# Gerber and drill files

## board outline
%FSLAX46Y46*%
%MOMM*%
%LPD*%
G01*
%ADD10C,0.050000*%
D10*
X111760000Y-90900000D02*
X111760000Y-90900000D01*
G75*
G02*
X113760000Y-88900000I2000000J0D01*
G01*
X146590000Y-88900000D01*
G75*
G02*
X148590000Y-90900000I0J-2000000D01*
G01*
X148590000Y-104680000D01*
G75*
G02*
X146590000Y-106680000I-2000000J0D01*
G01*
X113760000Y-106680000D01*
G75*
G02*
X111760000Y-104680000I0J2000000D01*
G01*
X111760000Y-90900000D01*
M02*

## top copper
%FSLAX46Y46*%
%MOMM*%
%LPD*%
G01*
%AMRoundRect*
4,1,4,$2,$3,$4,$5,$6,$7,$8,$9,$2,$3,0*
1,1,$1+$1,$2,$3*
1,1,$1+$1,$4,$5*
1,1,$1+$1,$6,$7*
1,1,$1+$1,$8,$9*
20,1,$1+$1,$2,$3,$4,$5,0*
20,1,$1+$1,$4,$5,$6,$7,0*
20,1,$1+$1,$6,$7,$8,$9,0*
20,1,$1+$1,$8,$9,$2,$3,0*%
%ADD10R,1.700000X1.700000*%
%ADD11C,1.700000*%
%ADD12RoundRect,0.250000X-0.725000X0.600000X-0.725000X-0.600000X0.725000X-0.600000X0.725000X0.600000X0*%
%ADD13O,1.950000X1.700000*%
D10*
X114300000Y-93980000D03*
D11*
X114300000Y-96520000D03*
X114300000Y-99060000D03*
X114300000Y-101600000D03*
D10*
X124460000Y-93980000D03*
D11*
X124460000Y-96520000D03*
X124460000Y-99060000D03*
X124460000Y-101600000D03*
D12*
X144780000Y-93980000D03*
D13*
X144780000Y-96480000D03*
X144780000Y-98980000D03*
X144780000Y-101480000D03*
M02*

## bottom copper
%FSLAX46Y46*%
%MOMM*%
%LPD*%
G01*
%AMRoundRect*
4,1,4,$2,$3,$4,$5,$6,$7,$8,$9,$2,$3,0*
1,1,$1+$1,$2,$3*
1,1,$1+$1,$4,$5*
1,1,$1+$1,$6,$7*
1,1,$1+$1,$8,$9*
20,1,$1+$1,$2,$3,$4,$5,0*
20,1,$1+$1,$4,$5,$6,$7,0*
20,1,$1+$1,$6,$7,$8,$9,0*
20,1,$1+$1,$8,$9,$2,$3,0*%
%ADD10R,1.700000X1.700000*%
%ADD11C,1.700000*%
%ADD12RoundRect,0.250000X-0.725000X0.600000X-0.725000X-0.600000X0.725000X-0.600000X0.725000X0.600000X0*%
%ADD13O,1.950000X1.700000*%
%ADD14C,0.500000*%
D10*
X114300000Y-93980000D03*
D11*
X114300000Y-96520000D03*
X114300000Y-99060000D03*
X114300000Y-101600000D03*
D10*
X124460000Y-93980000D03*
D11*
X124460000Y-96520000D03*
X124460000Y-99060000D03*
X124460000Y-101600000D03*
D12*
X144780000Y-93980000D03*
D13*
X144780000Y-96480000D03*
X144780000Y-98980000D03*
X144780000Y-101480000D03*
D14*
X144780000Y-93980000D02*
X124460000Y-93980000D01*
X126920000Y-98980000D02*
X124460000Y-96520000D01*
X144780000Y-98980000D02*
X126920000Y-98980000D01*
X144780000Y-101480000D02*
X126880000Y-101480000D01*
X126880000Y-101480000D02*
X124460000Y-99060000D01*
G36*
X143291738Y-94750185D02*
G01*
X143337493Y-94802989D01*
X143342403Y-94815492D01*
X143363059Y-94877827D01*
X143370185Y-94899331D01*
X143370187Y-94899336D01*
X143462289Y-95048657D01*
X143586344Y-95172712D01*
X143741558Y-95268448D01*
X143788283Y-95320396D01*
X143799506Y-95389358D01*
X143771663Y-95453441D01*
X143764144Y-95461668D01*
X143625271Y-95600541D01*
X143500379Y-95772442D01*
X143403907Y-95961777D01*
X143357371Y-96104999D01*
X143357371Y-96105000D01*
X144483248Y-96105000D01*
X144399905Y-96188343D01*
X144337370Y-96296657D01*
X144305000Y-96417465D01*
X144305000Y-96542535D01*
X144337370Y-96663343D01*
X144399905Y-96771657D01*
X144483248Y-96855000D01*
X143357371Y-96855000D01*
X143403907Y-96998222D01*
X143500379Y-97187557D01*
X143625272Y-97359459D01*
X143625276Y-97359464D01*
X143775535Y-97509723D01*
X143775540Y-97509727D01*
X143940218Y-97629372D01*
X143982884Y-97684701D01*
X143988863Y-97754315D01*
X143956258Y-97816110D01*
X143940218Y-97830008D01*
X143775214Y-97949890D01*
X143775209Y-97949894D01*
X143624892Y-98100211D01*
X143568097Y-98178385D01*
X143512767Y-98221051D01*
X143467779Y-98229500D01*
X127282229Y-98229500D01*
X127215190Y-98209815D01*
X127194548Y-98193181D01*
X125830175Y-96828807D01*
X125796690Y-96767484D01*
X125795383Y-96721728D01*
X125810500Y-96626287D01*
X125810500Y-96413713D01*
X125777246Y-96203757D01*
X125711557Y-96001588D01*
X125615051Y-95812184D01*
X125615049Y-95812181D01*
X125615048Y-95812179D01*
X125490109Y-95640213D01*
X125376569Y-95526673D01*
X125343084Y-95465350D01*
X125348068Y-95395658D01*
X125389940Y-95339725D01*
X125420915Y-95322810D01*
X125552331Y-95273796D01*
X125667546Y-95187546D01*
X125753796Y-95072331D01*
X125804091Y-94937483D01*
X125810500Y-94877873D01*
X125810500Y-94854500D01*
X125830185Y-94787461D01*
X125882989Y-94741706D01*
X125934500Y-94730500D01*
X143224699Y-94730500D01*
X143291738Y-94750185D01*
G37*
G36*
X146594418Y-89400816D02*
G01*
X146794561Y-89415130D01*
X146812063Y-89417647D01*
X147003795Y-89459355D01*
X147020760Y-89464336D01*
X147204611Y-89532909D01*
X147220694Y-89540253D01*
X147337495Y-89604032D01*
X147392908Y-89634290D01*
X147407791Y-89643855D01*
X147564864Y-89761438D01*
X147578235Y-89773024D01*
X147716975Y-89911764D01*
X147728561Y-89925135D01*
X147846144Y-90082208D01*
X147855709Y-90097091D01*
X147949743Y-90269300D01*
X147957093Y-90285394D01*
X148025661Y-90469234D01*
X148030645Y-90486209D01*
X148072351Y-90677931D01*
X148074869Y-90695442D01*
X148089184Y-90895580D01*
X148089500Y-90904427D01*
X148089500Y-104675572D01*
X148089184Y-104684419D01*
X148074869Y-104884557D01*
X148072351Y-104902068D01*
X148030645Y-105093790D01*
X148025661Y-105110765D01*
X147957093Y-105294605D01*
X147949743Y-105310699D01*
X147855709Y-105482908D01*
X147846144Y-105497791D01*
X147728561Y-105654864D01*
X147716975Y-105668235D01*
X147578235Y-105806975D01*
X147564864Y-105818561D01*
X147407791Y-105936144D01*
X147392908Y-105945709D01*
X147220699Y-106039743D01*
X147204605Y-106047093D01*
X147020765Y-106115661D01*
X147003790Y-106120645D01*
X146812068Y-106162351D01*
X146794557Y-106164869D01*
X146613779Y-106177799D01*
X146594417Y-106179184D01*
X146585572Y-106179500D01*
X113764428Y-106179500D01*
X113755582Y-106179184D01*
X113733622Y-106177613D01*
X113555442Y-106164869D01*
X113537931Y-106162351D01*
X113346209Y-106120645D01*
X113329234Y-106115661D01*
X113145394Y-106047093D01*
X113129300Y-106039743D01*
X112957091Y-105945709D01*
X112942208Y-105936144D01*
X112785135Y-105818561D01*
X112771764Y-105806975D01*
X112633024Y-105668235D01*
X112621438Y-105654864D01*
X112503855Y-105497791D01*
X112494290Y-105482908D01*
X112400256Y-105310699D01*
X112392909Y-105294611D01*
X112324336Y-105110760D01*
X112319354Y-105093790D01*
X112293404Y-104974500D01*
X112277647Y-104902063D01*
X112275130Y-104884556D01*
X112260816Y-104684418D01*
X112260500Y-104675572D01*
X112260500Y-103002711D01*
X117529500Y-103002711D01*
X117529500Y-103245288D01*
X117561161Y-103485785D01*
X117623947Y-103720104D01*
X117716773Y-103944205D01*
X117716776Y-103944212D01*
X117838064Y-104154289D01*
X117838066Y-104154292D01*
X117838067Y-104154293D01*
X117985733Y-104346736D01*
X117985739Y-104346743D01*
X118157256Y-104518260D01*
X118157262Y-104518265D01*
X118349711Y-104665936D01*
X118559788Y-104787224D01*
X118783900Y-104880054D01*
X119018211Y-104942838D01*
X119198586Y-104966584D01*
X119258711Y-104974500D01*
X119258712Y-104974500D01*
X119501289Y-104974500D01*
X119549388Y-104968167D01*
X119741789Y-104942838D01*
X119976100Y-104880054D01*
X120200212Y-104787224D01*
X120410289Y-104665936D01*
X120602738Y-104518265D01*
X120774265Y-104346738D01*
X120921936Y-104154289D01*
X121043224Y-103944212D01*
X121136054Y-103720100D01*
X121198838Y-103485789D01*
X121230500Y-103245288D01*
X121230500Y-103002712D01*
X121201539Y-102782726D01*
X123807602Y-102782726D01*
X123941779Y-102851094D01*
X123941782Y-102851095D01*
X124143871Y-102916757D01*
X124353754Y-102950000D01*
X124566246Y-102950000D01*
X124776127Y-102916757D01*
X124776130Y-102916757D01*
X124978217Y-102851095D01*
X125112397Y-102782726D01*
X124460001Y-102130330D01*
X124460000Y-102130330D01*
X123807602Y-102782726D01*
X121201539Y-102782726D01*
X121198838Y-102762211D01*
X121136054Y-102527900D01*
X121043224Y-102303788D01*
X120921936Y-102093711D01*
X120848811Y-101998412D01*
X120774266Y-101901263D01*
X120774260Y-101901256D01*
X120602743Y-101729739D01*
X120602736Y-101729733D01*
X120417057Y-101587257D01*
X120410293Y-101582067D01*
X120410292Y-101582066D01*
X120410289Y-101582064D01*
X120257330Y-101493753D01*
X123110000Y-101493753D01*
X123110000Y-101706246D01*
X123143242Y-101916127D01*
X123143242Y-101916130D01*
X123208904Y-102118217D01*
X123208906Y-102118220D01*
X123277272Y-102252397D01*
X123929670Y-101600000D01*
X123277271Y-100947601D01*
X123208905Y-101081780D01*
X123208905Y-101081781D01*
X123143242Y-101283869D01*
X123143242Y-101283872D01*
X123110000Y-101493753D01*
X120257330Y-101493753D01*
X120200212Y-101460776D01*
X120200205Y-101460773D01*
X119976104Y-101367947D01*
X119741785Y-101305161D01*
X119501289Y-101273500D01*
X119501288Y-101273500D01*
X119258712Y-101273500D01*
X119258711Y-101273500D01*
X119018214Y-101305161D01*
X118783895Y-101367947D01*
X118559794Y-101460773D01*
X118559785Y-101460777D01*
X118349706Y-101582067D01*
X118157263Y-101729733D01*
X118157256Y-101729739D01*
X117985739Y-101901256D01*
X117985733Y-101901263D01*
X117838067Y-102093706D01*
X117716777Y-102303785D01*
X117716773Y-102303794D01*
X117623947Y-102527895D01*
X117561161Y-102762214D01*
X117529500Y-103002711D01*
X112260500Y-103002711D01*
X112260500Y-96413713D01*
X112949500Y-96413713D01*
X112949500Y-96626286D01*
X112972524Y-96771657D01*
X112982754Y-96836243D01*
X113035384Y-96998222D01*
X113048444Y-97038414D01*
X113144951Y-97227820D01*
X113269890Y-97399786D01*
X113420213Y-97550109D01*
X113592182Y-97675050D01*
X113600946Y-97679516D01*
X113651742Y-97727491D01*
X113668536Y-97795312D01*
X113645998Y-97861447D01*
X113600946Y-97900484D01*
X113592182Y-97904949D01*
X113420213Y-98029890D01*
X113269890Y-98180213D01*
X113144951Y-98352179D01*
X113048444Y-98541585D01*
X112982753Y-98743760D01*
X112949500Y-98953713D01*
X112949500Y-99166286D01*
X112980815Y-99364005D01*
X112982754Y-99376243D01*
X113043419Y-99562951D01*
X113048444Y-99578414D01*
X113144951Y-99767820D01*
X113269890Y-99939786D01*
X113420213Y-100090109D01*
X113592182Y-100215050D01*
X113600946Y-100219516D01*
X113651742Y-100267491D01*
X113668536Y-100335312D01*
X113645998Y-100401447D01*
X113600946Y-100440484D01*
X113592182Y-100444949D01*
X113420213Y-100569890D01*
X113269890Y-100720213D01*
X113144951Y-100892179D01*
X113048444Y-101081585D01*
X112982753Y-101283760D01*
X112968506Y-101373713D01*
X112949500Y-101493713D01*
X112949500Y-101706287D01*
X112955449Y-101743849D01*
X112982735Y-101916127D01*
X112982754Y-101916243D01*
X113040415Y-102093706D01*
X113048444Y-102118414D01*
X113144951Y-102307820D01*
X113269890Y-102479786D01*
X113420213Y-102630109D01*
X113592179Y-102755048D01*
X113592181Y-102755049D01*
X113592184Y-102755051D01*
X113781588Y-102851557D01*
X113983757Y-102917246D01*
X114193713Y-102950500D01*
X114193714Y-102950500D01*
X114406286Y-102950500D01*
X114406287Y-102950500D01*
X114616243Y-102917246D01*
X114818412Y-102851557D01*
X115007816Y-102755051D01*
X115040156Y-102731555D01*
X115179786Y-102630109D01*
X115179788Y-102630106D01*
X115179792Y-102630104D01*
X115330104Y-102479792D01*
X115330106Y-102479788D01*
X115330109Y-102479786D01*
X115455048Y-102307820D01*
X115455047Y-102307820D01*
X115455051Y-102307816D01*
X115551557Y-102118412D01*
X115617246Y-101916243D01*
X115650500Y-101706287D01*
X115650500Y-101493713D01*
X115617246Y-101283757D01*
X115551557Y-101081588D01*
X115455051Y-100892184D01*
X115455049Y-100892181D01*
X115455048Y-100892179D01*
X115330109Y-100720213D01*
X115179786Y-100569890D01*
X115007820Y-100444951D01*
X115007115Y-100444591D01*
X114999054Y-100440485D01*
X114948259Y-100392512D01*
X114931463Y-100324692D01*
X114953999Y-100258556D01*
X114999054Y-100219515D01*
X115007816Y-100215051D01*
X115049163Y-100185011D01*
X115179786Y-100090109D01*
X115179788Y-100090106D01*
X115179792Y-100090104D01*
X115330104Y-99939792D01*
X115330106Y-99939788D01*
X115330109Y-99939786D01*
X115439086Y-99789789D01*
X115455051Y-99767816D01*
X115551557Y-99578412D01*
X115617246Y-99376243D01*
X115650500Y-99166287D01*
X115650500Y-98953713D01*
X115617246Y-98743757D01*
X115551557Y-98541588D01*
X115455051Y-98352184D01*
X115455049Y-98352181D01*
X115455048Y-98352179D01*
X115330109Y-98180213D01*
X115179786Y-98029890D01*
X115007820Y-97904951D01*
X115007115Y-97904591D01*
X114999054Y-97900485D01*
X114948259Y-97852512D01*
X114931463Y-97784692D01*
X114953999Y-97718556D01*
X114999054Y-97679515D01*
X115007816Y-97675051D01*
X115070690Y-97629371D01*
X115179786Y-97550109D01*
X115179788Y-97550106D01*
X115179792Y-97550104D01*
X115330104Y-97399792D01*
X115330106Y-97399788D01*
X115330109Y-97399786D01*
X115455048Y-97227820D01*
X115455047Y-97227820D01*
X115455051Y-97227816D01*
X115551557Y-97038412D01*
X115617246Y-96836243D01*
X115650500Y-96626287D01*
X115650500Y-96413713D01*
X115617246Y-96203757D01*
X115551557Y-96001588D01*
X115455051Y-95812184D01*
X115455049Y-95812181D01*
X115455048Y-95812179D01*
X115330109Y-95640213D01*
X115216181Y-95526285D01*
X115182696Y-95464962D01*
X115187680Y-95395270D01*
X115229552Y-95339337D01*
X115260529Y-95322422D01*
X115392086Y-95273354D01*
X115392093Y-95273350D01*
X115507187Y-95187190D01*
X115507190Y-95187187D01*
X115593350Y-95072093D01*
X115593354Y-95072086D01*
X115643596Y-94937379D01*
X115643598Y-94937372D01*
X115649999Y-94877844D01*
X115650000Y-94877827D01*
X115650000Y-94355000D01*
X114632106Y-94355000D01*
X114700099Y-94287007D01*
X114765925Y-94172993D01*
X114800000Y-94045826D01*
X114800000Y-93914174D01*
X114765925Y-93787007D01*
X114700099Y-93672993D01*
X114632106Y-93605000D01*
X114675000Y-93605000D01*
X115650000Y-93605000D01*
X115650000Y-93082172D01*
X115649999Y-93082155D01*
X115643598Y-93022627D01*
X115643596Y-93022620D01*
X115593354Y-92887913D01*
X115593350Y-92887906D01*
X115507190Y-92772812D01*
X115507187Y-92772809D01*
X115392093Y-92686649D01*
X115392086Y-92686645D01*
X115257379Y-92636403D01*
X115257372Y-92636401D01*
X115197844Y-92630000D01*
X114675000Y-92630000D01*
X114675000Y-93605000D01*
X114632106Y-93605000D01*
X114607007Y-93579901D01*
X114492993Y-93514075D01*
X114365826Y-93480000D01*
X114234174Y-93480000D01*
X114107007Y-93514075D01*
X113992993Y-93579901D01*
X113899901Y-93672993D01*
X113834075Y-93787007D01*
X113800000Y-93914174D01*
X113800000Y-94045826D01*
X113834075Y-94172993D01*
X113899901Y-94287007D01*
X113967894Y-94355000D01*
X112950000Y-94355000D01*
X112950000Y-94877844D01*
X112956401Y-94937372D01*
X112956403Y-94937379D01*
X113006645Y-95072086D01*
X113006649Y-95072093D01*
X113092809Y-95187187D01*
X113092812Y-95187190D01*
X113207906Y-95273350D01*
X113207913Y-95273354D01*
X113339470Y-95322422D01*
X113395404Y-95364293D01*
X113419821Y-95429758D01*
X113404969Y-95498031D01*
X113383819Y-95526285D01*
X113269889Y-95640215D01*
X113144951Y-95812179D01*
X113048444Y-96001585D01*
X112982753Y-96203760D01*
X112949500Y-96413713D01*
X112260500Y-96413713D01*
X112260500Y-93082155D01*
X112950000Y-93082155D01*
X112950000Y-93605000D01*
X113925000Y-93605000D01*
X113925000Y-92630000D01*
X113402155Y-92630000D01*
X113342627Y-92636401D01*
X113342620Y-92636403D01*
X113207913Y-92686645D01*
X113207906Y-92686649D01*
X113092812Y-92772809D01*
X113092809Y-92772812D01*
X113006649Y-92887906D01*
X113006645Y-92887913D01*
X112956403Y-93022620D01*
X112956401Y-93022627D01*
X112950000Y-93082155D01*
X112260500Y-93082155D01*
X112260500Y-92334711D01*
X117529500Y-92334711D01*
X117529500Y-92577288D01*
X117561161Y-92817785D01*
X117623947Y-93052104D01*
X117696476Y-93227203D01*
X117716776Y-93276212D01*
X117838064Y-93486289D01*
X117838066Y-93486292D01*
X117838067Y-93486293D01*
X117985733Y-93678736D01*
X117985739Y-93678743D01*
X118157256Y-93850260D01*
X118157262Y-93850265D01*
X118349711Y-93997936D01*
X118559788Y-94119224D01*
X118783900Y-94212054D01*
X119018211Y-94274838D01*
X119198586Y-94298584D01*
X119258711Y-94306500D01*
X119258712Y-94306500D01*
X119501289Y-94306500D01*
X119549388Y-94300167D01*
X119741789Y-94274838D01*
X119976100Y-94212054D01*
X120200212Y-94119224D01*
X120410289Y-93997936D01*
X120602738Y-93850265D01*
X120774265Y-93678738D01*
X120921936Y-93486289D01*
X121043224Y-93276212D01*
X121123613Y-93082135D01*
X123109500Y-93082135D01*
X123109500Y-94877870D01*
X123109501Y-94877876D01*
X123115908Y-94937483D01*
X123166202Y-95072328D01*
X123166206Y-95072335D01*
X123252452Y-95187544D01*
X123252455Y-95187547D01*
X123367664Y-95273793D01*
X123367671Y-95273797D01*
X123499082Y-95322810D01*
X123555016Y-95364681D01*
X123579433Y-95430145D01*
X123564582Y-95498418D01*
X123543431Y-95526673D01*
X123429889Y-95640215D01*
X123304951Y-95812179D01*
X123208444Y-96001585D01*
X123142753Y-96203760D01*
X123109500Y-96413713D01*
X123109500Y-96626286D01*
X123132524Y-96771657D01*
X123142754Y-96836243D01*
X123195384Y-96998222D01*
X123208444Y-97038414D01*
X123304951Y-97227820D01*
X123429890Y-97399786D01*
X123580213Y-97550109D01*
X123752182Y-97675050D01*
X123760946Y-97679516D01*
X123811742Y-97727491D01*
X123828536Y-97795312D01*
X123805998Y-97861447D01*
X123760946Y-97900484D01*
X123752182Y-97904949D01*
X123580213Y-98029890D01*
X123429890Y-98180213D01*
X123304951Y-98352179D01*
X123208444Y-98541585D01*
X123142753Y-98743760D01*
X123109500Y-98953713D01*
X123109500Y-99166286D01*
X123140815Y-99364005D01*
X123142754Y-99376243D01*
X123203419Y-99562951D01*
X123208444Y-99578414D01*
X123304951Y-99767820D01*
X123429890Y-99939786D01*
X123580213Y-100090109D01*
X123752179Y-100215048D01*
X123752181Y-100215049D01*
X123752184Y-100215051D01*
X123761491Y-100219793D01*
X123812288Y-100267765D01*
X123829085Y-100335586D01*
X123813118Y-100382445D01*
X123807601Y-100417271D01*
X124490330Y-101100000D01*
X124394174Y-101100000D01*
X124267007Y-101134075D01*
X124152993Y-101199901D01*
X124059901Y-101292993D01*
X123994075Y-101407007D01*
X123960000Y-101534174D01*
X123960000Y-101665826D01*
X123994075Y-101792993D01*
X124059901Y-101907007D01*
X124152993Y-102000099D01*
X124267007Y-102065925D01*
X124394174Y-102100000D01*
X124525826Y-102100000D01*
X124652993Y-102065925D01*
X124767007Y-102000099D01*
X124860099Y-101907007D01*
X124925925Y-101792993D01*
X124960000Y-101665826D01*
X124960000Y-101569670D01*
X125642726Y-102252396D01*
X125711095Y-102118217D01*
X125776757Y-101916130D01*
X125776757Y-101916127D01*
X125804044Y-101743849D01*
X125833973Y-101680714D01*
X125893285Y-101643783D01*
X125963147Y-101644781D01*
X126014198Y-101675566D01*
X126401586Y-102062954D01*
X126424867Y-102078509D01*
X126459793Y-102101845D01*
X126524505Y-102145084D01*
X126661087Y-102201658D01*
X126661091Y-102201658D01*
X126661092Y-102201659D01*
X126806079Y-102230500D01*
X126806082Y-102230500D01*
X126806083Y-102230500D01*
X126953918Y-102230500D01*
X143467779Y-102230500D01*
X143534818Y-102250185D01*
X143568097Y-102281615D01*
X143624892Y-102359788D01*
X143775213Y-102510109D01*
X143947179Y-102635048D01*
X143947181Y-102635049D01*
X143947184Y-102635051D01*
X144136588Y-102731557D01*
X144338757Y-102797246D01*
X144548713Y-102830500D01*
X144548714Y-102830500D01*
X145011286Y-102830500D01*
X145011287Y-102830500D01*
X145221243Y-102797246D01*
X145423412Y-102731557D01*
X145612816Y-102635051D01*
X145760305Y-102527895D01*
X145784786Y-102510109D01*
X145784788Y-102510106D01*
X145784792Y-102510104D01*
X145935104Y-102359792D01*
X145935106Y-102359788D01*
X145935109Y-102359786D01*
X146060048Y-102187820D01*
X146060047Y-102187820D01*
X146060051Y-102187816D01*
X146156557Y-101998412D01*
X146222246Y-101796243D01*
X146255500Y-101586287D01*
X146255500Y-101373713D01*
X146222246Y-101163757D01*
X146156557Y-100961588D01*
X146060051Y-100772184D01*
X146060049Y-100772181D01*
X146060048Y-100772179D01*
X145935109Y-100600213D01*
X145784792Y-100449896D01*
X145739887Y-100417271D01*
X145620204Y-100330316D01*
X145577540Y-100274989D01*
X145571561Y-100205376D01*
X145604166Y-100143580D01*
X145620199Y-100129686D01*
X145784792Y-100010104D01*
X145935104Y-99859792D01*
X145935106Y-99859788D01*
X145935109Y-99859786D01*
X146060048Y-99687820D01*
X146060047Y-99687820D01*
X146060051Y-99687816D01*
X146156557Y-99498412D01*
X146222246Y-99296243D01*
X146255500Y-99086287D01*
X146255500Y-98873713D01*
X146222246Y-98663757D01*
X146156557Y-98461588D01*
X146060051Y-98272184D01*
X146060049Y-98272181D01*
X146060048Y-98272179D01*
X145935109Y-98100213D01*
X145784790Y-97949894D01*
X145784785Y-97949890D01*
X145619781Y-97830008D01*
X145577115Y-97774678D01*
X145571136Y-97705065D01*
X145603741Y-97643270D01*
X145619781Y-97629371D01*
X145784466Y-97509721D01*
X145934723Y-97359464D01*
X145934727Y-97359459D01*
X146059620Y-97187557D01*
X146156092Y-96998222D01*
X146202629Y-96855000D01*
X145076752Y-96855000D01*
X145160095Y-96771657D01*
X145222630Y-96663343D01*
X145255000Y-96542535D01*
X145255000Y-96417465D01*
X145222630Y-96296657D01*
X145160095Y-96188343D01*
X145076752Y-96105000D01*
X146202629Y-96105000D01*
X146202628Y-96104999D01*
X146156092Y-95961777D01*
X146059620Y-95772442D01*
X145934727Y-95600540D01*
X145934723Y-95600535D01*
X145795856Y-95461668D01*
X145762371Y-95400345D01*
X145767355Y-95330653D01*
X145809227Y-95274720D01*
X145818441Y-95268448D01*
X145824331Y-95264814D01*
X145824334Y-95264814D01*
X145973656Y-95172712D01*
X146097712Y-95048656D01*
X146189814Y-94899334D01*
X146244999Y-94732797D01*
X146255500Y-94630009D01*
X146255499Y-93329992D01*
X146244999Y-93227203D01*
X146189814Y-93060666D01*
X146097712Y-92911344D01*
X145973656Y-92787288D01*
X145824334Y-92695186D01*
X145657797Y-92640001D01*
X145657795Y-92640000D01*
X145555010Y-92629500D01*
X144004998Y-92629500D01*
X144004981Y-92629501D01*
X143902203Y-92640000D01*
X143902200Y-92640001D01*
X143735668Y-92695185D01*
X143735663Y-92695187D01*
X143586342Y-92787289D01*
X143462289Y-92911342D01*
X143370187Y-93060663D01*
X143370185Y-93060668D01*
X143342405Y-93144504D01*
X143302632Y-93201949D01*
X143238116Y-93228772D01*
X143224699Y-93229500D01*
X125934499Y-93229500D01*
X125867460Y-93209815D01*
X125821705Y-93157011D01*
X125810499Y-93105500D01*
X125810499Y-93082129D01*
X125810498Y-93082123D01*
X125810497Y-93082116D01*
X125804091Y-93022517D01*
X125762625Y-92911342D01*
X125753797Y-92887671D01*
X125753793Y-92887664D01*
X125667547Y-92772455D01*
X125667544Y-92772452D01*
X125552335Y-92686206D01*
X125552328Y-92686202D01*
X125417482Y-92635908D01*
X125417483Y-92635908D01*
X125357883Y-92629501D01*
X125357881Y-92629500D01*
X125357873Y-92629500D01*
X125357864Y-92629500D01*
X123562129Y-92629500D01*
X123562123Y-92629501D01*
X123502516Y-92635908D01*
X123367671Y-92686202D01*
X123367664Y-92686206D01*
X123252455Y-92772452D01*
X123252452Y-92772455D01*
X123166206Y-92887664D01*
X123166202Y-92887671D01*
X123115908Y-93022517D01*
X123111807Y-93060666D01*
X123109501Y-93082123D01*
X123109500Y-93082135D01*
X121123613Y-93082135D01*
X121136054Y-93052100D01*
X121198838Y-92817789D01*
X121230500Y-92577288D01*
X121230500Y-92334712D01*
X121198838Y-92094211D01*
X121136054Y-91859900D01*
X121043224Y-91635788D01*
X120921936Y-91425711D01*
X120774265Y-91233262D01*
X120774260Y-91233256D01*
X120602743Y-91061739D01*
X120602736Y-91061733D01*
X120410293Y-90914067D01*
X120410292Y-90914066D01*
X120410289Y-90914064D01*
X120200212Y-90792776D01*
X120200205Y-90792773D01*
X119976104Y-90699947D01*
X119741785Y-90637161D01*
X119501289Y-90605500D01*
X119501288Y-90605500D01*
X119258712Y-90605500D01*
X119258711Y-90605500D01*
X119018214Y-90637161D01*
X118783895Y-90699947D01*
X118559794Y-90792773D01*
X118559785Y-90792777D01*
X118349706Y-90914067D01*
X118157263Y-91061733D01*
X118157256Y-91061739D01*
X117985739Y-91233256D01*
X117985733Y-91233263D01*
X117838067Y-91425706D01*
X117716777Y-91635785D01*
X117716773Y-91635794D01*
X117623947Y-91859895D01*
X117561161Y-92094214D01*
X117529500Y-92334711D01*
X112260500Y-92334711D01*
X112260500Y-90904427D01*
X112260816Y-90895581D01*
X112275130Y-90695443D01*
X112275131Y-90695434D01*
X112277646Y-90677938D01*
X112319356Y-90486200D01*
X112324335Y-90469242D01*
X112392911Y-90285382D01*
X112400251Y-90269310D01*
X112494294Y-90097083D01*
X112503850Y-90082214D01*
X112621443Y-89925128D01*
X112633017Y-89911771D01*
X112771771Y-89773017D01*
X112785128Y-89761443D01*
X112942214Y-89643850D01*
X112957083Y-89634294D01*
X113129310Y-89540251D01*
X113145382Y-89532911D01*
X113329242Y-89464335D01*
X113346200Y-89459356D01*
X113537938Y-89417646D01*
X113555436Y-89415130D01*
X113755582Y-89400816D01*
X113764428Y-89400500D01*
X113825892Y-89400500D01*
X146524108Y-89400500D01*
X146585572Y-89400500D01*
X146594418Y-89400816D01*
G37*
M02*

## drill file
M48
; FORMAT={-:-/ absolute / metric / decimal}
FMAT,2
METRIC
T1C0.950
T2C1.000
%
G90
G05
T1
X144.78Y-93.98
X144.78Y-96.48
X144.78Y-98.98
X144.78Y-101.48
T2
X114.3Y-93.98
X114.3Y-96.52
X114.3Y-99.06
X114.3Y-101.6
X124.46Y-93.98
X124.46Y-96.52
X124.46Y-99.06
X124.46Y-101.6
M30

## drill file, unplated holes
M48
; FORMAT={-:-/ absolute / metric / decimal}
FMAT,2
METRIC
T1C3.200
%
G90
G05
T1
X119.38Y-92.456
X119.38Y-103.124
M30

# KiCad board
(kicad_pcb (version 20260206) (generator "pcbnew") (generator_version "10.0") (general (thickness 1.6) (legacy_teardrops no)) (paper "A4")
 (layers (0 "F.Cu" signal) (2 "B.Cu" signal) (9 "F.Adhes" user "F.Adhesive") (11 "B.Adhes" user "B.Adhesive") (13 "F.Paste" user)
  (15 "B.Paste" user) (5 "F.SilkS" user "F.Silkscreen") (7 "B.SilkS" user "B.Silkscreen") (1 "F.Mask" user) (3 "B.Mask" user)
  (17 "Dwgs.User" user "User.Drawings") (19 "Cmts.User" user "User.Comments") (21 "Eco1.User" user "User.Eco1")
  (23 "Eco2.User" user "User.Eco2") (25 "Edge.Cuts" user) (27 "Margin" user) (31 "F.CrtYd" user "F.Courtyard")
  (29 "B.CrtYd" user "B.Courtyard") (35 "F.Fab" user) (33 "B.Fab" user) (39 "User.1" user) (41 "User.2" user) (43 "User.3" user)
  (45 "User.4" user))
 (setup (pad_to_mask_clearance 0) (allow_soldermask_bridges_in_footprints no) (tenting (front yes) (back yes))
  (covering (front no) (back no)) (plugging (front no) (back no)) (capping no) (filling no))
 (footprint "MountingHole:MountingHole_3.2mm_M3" (layer "F.Cu") (at 119.38 92.456)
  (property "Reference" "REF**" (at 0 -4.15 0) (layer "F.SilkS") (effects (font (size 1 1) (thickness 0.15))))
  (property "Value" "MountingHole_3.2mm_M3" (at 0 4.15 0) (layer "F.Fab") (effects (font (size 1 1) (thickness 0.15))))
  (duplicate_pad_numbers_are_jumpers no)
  (pad "" np_thru_hole circle (at 0 0) (size 3.2 3.2) (drill 3.2) (layers "*.Cu" "*.Mask")))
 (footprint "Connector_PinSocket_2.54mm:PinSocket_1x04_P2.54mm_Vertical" (layer "F.Cu") (at 114.3 93.98)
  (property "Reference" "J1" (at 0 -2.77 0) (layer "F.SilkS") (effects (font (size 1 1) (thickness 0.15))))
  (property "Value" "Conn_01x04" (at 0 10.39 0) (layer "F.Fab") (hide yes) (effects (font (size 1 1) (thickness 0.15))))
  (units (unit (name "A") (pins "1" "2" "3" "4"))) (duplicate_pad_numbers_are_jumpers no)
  (pad "1" thru_hole rect (at 0 0) (size 1.7 1.7) (drill 1) (layers "*.Cu" "*.Mask") (remove_unused_layers no) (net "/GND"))
  (pad "2" thru_hole circle (at 0 2.54) (size 1.7 1.7) (drill 1) (layers "*.Cu" "*.Mask") (remove_unused_layers no) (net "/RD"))
  (pad "3" thru_hole circle (at 0 5.08) (size 1.7 1.7) (drill 1) (layers "*.Cu" "*.Mask") (remove_unused_layers no) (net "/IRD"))
  (pad "4" thru_hole circle (at 0 7.62) (size 1.7 1.7) (drill 1) (layers "*.Cu" "*.Mask") (remove_unused_layers no) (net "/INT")))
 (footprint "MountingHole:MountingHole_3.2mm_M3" (layer "F.Cu") (at 119.38 103.124)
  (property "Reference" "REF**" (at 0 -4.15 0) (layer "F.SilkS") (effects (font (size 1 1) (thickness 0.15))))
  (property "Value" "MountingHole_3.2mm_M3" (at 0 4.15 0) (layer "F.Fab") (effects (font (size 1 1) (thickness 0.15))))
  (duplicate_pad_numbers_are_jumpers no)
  (pad "" np_thru_hole circle (at 0 0) (size 3.2 3.2) (drill 3.2) (layers "*.Cu" "*.Mask")))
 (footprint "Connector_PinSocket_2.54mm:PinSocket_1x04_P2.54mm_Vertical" (layer "F.Cu") (at 124.46 93.98)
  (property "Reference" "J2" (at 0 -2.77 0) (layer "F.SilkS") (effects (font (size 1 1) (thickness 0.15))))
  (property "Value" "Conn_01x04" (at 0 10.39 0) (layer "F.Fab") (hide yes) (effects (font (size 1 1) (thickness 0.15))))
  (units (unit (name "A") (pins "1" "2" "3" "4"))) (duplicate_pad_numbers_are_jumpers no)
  (pad "1" thru_hole rect (at 0 0) (size 1.7 1.7) (drill 1) (layers "*.Cu" "*.Mask") (remove_unused_layers no) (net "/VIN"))
  (pad "2" thru_hole circle (at 0 2.54) (size 1.7 1.7) (drill 1) (layers "*.Cu" "*.Mask") (remove_unused_layers no) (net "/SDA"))
  (pad "3" thru_hole circle (at 0 5.08) (size 1.7 1.7) (drill 1) (layers "*.Cu" "*.Mask") (remove_unused_layers no) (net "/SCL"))
  (pad "4" thru_hole circle (at 0 7.62) (size 1.7 1.7) (drill 1) (layers "*.Cu" "*.Mask") (remove_unused_layers no) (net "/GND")))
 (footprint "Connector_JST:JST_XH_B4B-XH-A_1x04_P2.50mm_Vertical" (layer "F.Cu") (at 144.78 93.98 -90)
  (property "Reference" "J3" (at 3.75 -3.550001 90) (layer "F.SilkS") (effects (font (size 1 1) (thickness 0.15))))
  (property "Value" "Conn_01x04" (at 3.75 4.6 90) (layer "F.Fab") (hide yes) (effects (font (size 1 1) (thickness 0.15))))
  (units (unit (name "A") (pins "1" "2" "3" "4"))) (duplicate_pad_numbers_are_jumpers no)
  (pad "1" thru_hole roundrect (at 0 0 270) (size 1.7 1.95) (drill 0.95) (layers "*.Cu" "*.Mask") (remove_unused_layers no)
   (roundrect_rratio 0.147059) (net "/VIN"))
  (pad "2" thru_hole oval (at 2.5 0 270) (size 1.7 1.95) (drill 0.95) (layers "*.Cu" "*.Mask") (remove_unused_layers no) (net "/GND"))
  (pad "3" thru_hole oval (at 5 0 270) (size 1.7 1.95) (drill 0.95) (layers "*.Cu" "*.Mask") (remove_unused_layers no) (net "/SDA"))
  (pad "4" thru_hole oval (at 7.5 0 270) (size 1.7 1.95) (drill 0.95) (layers "*.Cu" "*.Mask") (remove_unused_layers no) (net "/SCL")))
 (gr_rect (start 111.76 88.9) (end 148.59 106.68) (radius 2) (stroke (width 0.05) (type solid)) (fill no) (layer "Edge.Cuts"))
 (segment (start 144.78 93.98) (end 124.46 93.98) (width 0.5) (layer "B.Cu") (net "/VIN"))
 (segment (start 126.92 98.98) (end 124.46 96.52) (width 0.5) (layer "B.Cu") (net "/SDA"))
 (segment (start 144.78 98.98) (end 126.92 98.98) (width 0.5) (layer "B.Cu") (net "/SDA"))
 (segment (start 144.78 101.48) (end 126.88 101.48) (width 0.5) (layer "B.Cu") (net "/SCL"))
 (segment (start 126.88 101.48) (end 124.46 99.06) (width 0.5) (layer "B.Cu") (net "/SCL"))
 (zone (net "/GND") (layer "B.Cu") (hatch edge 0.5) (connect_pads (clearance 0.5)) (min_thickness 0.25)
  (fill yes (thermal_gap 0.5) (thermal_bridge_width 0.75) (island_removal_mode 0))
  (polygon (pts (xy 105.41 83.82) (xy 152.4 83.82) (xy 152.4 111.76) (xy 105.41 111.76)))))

